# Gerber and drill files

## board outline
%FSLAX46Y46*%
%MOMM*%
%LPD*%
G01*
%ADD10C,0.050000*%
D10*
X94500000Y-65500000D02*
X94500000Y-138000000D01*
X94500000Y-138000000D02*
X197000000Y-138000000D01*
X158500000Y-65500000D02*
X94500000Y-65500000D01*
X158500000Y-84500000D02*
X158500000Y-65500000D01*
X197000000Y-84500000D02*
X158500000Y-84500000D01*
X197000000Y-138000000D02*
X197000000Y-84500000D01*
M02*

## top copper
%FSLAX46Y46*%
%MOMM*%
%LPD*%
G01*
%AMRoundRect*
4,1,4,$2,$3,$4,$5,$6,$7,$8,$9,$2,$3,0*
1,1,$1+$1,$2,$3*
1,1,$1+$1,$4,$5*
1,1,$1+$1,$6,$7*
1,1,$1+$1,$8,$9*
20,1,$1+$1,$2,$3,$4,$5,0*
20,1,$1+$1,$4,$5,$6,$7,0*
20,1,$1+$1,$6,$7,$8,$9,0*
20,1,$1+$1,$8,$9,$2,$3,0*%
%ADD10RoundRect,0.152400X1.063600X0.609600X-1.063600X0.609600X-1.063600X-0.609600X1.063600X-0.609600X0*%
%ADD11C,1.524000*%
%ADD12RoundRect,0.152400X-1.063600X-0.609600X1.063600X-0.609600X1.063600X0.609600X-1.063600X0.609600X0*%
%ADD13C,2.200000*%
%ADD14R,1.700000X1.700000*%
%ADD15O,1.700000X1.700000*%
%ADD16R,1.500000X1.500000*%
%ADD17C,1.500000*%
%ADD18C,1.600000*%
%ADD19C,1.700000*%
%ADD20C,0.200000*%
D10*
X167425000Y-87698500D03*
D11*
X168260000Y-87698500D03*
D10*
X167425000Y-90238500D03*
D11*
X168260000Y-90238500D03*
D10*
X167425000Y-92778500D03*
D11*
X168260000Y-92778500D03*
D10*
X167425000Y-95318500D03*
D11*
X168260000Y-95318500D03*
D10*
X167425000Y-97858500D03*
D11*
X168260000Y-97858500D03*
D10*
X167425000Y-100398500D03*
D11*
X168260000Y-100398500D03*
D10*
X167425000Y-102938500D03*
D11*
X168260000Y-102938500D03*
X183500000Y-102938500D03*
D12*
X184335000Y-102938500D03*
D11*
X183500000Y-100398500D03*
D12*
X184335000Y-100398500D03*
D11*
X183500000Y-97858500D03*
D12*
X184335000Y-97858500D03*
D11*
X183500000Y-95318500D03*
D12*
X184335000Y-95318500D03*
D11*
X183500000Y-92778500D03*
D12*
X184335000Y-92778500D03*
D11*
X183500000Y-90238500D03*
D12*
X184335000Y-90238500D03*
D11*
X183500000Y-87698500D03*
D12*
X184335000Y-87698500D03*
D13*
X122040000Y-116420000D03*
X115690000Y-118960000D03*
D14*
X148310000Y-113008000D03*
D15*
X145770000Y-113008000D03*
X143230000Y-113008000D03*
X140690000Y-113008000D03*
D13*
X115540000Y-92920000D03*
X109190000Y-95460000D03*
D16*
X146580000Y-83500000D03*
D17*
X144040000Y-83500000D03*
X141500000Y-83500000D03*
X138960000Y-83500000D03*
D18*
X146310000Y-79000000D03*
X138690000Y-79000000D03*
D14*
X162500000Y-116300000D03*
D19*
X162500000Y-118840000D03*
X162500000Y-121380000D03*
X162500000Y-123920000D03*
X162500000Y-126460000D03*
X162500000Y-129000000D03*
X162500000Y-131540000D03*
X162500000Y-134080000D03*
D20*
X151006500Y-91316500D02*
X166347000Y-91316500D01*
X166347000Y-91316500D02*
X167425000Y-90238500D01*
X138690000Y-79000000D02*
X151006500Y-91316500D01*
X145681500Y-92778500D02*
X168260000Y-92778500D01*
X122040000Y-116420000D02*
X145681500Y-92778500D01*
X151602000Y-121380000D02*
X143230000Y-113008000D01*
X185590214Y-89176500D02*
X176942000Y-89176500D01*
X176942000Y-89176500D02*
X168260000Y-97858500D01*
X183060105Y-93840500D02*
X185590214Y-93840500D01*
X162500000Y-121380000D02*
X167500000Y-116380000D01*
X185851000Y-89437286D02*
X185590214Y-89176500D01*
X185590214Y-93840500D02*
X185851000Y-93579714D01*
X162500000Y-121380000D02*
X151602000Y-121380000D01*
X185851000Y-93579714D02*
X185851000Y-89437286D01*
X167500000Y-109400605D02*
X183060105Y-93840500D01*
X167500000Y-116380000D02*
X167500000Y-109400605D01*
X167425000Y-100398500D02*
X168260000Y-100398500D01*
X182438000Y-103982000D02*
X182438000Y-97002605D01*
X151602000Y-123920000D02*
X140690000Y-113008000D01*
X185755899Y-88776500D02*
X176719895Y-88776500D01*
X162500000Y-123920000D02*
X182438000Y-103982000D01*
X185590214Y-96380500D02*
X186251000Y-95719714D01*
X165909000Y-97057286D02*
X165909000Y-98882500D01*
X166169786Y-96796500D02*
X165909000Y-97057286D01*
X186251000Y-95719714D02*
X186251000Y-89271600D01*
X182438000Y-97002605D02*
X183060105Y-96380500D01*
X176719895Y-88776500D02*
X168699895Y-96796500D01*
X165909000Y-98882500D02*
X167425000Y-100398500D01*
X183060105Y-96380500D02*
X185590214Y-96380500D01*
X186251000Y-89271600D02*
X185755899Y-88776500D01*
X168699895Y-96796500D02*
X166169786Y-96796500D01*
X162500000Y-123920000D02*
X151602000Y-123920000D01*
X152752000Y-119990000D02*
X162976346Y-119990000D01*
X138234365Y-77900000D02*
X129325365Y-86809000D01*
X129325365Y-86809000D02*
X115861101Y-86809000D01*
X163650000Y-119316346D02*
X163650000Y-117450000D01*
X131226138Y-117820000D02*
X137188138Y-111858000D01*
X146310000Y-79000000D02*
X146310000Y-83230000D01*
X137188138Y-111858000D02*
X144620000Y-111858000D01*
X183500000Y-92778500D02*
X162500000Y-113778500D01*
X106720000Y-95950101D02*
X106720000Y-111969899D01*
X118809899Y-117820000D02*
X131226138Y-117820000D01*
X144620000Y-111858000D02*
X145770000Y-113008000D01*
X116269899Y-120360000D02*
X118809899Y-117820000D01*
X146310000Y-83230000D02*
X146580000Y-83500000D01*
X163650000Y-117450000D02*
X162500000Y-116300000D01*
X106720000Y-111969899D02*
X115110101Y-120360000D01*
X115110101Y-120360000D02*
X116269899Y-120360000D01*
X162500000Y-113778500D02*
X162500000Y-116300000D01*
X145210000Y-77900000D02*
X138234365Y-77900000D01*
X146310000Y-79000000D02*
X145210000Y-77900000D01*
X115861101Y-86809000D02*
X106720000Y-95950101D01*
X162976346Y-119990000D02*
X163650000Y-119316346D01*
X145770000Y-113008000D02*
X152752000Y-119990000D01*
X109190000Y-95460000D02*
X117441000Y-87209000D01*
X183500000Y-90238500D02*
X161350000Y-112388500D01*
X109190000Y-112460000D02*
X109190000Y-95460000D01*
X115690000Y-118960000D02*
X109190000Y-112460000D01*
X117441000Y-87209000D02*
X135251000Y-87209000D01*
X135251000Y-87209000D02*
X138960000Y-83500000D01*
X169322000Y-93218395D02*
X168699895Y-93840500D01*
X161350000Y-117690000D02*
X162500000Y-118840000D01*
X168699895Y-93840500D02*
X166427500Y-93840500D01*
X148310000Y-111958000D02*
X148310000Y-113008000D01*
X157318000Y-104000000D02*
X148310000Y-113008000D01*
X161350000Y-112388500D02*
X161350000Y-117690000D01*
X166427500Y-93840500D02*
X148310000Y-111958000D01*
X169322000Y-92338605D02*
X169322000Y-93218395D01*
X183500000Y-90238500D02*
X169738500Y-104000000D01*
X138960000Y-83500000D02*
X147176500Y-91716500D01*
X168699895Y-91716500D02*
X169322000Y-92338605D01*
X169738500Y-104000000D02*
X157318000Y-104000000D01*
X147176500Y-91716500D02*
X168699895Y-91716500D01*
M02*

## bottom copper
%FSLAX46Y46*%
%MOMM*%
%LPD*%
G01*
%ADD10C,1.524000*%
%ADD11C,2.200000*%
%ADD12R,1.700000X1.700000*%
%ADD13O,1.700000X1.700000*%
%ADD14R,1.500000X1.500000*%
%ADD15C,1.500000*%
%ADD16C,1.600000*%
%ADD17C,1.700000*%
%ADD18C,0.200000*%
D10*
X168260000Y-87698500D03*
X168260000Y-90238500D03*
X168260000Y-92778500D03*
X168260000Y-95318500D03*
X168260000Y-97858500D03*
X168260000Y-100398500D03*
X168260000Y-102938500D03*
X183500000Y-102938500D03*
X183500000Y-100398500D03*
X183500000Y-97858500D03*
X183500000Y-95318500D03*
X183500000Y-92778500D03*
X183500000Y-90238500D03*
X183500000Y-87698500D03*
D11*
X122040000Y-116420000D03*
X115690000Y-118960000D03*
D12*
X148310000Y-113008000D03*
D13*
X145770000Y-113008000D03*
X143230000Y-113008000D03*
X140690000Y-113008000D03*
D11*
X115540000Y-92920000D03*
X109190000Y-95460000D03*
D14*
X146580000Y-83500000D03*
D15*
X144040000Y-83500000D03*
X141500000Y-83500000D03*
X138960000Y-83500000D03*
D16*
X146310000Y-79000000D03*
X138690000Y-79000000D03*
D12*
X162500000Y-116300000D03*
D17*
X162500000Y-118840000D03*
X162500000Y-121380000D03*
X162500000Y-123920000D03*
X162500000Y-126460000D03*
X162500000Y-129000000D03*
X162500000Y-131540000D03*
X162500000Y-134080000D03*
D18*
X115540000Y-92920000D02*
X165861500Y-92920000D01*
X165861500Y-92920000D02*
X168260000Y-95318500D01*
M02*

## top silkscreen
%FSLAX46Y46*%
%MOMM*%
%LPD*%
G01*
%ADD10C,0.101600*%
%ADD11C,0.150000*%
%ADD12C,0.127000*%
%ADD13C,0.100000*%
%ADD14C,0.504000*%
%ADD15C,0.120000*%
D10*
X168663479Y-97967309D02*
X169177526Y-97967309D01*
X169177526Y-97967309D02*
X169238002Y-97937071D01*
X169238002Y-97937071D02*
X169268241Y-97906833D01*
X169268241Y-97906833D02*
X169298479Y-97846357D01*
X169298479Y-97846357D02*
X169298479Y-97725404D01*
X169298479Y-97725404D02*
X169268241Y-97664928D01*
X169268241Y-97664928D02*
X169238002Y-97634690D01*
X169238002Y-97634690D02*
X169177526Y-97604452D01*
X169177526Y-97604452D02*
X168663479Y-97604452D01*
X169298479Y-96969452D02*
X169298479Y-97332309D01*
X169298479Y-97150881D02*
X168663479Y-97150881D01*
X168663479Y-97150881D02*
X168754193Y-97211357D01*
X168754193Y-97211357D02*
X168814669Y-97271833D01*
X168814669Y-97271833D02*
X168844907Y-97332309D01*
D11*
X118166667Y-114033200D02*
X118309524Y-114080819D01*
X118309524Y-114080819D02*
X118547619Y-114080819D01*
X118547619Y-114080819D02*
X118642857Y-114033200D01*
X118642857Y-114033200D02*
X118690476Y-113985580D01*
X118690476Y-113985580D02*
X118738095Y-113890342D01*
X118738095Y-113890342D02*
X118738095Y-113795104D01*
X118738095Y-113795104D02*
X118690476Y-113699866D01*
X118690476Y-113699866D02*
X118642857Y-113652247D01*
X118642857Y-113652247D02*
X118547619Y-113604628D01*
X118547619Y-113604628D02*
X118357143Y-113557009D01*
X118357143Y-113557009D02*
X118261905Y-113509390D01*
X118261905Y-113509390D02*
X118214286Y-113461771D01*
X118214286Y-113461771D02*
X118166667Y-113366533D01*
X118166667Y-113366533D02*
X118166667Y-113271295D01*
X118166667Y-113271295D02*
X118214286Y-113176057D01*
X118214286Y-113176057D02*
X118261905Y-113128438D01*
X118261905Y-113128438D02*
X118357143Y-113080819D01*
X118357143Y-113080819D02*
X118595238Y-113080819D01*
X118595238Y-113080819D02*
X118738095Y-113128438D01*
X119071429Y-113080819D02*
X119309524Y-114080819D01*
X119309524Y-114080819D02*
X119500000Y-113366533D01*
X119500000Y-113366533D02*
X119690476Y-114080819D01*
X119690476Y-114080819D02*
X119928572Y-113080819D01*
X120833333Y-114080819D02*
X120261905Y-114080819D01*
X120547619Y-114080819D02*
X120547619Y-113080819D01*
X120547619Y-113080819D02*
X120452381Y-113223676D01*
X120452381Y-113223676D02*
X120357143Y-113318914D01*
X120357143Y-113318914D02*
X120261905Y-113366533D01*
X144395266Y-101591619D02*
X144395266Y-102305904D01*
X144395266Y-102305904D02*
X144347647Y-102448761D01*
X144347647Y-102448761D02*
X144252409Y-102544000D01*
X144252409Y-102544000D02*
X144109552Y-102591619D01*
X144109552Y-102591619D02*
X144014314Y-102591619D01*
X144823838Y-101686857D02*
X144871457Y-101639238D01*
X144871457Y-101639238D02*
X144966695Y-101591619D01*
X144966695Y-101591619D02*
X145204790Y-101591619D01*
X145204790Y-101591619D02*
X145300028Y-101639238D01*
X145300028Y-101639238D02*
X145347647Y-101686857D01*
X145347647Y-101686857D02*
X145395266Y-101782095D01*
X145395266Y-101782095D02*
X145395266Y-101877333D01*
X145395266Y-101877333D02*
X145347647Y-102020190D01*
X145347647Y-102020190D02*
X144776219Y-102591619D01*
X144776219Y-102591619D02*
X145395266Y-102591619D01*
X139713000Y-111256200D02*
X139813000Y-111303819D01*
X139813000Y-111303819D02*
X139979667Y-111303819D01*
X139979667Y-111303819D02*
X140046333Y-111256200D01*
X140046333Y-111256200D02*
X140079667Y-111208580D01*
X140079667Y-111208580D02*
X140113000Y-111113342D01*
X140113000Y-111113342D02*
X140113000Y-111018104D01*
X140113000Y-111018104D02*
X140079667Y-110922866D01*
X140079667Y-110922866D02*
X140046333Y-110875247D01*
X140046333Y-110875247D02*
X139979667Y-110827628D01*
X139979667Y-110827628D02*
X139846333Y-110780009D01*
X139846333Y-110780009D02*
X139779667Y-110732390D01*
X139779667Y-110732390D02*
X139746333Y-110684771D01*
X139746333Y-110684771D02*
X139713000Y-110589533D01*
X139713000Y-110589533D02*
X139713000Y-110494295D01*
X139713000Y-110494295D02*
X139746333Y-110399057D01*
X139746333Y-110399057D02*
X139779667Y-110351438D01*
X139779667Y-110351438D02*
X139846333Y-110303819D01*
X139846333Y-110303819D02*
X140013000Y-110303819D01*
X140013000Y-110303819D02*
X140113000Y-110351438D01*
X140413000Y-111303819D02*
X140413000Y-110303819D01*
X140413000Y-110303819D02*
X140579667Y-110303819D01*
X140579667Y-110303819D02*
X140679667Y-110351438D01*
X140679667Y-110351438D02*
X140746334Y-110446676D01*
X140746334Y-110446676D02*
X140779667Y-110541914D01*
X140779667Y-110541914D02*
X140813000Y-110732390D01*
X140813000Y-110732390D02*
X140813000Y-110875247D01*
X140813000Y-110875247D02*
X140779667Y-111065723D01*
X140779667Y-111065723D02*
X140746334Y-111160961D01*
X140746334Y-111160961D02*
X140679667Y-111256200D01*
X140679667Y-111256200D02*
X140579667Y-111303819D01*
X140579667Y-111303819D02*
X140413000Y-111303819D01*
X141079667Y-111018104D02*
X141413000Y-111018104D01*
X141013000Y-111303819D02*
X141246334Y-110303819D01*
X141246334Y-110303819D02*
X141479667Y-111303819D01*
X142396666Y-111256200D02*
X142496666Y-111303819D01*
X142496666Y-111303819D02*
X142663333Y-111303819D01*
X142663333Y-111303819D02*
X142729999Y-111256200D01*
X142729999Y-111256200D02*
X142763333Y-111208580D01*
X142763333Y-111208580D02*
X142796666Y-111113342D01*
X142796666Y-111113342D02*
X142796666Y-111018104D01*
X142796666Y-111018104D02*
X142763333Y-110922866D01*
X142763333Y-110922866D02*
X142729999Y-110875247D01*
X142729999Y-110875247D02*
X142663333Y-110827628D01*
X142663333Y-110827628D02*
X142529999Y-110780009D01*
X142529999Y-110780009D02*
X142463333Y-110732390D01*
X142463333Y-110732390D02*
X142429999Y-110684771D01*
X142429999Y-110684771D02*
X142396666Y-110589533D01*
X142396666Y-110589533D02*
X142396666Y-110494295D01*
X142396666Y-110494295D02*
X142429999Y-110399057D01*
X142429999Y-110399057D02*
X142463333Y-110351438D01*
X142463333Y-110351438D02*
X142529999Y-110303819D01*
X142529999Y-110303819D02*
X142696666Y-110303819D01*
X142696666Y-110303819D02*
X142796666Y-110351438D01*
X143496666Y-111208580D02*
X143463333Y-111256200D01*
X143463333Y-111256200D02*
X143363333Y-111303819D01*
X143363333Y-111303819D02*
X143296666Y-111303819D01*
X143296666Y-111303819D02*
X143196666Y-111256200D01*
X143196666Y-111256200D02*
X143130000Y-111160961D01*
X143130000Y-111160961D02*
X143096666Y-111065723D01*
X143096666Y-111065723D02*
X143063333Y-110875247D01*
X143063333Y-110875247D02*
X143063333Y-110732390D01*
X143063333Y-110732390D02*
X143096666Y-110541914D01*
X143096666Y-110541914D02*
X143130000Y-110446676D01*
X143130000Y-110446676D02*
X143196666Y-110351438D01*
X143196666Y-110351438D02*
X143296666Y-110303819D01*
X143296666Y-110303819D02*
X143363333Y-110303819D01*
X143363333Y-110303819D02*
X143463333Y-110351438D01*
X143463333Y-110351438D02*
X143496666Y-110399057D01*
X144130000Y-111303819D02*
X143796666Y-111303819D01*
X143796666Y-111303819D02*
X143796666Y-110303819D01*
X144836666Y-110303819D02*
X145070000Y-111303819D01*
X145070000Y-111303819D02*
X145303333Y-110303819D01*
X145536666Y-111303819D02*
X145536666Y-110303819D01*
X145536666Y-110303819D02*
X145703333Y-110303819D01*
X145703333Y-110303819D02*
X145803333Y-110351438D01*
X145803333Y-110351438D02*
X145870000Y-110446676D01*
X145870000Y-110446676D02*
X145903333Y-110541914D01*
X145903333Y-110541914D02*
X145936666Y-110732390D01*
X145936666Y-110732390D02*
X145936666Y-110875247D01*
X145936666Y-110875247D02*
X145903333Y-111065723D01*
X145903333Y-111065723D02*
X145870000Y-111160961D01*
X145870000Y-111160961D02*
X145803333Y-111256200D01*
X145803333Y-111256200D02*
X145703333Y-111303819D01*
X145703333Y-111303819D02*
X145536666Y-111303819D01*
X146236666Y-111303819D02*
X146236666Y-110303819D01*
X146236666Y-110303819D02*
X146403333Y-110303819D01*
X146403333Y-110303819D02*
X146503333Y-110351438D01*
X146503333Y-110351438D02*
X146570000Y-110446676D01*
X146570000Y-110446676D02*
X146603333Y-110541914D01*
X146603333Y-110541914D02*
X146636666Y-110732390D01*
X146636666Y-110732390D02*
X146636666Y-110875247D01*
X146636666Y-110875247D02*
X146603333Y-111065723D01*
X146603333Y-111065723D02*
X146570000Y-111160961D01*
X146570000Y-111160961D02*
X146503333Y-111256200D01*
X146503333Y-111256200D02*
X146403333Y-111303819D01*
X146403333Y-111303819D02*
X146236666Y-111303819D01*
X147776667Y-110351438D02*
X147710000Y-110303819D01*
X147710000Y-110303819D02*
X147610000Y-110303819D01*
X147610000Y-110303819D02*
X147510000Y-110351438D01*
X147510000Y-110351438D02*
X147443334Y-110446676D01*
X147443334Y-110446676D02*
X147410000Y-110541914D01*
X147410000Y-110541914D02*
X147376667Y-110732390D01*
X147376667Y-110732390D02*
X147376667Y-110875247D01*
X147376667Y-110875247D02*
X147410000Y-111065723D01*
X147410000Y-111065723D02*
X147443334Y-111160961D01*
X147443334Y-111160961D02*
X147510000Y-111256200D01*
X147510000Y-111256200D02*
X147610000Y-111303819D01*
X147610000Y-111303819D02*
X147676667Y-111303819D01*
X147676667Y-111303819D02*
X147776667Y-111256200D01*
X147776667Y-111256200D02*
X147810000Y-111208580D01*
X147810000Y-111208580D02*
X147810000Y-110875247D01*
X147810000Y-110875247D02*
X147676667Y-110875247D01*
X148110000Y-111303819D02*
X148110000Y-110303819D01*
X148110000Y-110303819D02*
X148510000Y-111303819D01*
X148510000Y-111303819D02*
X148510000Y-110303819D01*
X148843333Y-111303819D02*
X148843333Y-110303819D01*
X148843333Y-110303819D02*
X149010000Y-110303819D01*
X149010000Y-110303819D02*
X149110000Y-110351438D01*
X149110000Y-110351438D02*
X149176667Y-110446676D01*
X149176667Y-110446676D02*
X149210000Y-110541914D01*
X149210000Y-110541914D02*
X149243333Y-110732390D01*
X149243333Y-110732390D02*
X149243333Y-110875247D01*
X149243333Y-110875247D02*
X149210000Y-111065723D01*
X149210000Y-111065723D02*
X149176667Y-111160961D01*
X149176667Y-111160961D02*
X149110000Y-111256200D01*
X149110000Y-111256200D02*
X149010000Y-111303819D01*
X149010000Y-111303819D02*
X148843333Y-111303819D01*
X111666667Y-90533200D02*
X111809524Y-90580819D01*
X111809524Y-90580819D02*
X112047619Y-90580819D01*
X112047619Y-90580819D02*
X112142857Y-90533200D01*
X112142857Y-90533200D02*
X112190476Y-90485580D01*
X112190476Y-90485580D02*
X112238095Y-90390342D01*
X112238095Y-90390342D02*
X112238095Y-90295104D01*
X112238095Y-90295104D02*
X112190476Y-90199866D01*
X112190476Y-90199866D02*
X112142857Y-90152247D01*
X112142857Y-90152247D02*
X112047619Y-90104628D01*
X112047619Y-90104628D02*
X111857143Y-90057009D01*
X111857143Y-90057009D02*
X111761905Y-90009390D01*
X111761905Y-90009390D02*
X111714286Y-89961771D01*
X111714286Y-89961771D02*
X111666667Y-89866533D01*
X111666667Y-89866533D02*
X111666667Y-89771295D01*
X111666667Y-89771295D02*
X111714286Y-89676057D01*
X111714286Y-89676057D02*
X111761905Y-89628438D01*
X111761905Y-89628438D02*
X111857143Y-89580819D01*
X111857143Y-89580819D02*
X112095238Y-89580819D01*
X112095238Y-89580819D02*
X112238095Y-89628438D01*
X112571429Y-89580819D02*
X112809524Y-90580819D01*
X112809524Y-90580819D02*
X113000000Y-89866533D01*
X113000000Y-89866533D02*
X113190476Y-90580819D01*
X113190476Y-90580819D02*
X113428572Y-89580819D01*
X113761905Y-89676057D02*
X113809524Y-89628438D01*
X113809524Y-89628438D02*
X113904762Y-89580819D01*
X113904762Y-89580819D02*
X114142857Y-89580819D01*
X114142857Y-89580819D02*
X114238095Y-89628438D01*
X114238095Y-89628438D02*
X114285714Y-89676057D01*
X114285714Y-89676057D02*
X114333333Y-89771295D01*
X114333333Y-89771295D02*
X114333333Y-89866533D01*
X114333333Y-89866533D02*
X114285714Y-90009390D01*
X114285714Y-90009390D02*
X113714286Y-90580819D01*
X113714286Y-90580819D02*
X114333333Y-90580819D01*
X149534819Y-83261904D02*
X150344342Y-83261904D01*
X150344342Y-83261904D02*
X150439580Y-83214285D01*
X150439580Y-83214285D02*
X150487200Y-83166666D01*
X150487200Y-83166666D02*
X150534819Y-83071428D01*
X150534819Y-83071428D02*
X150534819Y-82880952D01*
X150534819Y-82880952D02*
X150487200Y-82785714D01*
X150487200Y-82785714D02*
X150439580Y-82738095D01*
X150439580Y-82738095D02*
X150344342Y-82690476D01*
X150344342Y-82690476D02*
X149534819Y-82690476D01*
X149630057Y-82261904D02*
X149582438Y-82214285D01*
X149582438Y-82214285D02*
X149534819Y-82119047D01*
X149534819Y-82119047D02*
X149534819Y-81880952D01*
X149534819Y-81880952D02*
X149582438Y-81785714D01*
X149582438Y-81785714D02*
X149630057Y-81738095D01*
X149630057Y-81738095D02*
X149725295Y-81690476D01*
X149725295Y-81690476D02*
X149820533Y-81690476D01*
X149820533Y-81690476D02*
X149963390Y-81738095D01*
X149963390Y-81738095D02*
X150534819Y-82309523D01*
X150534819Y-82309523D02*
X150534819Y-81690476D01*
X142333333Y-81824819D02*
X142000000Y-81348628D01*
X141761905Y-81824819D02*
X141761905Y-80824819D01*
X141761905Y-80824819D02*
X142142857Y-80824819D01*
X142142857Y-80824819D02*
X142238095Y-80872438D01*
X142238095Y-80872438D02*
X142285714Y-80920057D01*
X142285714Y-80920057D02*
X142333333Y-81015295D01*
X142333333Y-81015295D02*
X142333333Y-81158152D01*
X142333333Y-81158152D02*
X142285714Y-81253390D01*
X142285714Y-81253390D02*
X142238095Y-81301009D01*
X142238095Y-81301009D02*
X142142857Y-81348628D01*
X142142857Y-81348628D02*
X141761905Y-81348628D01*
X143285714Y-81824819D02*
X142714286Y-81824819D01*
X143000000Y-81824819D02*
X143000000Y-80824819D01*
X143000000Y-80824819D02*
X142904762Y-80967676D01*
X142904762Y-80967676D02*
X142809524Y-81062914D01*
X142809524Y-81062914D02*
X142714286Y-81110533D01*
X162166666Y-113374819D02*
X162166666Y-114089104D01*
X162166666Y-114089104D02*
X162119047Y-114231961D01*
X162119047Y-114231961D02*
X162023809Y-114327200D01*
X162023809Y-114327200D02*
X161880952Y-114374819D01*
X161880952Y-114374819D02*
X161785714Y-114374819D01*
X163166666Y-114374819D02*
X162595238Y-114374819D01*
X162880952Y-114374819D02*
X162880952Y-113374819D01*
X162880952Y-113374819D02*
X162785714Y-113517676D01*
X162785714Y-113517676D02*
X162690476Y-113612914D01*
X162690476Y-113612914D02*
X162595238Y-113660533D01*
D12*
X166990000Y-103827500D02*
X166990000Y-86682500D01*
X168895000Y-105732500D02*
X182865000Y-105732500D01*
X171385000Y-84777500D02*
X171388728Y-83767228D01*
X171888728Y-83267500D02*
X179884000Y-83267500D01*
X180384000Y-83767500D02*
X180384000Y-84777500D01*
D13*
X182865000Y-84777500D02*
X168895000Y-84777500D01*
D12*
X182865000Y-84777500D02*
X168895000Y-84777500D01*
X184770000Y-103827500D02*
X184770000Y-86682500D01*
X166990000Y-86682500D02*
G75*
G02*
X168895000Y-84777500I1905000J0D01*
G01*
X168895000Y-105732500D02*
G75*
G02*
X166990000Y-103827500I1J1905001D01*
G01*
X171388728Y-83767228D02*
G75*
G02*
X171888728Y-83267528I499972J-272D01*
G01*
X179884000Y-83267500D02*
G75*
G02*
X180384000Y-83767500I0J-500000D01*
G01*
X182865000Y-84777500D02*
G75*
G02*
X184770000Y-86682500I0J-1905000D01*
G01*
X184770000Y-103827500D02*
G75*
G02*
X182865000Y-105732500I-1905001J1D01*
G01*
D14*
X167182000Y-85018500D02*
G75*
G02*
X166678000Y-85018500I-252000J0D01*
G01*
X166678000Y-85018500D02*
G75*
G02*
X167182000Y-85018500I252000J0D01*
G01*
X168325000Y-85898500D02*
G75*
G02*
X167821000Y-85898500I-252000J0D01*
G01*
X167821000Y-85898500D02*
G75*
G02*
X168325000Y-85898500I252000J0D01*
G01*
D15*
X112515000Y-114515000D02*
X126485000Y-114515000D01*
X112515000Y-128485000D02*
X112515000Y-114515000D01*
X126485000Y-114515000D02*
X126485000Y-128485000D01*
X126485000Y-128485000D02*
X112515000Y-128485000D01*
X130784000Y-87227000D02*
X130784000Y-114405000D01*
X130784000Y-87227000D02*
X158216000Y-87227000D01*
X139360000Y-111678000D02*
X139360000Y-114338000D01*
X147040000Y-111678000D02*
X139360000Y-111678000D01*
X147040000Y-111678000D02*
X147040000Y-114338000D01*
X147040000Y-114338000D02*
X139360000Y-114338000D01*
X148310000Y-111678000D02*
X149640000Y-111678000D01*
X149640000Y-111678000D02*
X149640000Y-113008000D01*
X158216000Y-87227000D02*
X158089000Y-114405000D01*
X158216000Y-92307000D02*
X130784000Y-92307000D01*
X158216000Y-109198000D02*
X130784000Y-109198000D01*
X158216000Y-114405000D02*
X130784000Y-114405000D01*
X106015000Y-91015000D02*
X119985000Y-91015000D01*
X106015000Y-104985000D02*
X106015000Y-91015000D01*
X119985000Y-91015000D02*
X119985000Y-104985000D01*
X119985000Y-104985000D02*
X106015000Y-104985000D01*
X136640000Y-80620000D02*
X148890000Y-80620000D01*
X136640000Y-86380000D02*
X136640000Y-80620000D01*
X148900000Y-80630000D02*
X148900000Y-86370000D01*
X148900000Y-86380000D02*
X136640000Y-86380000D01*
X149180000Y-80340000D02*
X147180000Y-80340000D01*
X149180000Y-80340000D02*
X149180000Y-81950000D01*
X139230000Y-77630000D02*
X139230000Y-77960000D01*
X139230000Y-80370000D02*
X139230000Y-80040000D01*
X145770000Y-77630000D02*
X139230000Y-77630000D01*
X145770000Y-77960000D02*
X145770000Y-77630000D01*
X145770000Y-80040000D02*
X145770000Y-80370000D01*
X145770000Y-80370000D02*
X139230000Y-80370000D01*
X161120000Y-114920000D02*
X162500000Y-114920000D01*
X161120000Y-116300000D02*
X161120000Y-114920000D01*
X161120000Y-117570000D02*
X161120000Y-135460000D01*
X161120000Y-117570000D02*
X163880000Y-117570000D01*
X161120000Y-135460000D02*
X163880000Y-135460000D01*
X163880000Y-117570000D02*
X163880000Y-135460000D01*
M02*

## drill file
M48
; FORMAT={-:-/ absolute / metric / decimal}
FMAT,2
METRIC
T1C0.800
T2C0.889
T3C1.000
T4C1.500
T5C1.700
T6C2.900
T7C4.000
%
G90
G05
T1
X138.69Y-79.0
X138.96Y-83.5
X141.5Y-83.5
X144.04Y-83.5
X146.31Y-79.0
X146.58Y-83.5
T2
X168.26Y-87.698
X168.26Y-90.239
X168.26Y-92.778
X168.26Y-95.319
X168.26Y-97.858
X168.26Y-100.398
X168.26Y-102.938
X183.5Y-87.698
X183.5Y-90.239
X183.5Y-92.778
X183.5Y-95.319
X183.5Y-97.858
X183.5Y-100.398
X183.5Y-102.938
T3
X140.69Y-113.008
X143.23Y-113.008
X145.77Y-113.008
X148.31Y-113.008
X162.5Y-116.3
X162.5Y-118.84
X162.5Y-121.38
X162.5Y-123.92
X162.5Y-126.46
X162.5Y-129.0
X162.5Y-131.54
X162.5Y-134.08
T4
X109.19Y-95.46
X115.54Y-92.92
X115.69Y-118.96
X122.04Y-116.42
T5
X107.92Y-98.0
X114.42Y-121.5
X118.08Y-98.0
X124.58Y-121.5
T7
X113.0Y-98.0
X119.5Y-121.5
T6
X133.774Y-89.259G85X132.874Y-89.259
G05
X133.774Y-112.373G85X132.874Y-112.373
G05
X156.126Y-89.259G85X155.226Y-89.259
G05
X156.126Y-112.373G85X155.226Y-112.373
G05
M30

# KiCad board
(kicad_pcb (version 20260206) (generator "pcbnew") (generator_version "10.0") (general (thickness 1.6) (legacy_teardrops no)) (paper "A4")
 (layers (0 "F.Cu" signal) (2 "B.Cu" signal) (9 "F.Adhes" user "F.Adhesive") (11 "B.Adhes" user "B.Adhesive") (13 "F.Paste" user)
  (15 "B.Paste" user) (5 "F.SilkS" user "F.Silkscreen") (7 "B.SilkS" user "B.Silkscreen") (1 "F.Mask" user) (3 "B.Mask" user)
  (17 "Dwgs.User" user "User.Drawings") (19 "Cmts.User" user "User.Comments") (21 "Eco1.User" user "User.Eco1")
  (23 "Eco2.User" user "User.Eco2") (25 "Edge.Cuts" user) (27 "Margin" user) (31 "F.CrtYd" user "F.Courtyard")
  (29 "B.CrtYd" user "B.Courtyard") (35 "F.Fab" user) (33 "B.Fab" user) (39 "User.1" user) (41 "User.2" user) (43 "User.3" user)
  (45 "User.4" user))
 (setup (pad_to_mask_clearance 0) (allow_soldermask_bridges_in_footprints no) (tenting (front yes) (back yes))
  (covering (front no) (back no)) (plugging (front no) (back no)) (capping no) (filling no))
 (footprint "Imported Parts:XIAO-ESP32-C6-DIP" (layer "F.Cu") (at 175.88 95.3185 90)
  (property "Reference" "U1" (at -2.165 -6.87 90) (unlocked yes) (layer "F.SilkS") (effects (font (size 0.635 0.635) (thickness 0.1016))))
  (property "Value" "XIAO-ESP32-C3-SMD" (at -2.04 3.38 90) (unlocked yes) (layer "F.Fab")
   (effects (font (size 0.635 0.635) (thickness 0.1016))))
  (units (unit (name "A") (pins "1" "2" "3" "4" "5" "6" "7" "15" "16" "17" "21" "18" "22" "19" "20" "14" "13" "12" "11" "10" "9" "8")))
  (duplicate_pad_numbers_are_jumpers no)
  (fp_line (start -8.509 -8.89) (end 8.636 -8.89) (stroke (width 0.127) (type solid)) (layer "F.SilkS"))
  (fp_line (start -10.414 -6.985) (end -10.414 6.985) (stroke (width 0.127) (type solid)) (layer "F.SilkS"))
  (fp_line (start 10.541 -4.495) (end 11.551272 -4.491272) (stroke (width 0.127) (type solid)) (layer "F.SilkS"))
  (fp_line (start 12.051 -3.991272) (end 12.051 4.004) (stroke (width 0.127) (type solid)) (layer "F.SilkS"))
  (fp_line (start 11.551 4.504) (end 10.541 4.504) (stroke (width 0.127) (type solid)) (layer "F.SilkS"))
  (fp_line (start 10.541 6.985) (end 10.541 -6.985) (stroke (width 0.1) (type solid)) (layer "F.SilkS"))
  (fp_line (start 10.541 6.985) (end 10.541 -6.985) (stroke (width 0.127) (type solid)) (layer "F.SilkS"))
  (fp_line (start -8.509 8.89) (end 8.636 8.89) (stroke (width 0.127) (type solid)) (layer "F.SilkS"))
  (fp_arc (start 8.636 -8.89) (mid 9.983038 -8.332038) (end 10.541 -6.985) (stroke (width 0.127) (type solid)) (layer "F.SilkS"))
  (fp_arc (start -10.414 -6.985) (mid -9.856038 -8.332038) (end -8.509 -8.89) (stroke (width 0.127) (type solid)) (layer "F.SilkS"))
  (fp_arc (start 11.551272 -4.491272) (mid 11.904644 -4.344724) (end 12.051 -3.991272) (stroke (width 0.127) (type default))
   (layer "F.SilkS"))
  (fp_arc (start 12.051 4.004) (mid 11.904553 4.357553) (end 11.551 4.504) (stroke (width 0.127) (type default)) (layer "F.SilkS"))
  (fp_arc (start 10.541 6.985) (mid 9.983038 8.332038) (end 8.636 8.89) (stroke (width 0.127) (type solid)) (layer "F.SilkS"))
  (fp_arc (start -8.509 8.89) (mid -9.856038 8.332038) (end -10.414 6.985) (stroke (width 0.127) (type solid)) (layer "F.SilkS"))
  (fp_circle (center 10.3 -8.95) (end 10.554 -8.95) (stroke (width 0.5) (type solid)) (fill yes) (layer "F.SilkS"))
  (fp_circle (center 9.42 -7.807) (end 9.674 -7.807) (stroke (width 0.5) (type solid)) (fill yes) (layer "F.SilkS"))
  (pad "1" smd roundrect (at 7.62 -8.455 180) (size 2.432 1.524) (layers "F.Cu" "F.Mask") (roundrect_rratio 0.1)
   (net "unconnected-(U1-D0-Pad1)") (thermal_bridge_angle 45))
  (pad "1" thru_hole circle (at 7.62 -7.62 180) (size 1.524 1.524) (drill 0.889) (layers "*.Cu" "*.Mask") (remove_unused_layers no)
   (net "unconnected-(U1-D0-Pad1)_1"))
  (pad "2" smd roundrect (at 5.08 -8.455 180) (size 2.432 1.524) (layers "F.Cu" "F.Mask") (roundrect_rratio 0.1) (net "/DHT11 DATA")
   (thermal_bridge_angle 45))
  (pad "2" thru_hole circle (at 5.08 -7.62 180) (size 1.524 1.524) (drill 0.889) (layers "*.Cu" "*.Mask") (remove_unused_layers no)
   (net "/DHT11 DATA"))
  (pad "3" smd roundrect (at 2.54 -8.455 180) (size 2.432 1.524) (layers "F.Cu" "F.Mask") (roundrect_rratio 0.1) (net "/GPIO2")
   (thermal_bridge_angle 45))
  (pad "3" thru_hole circle (at 2.54 -7.62 180) (size 1.524 1.524) (drill 0.889) (layers "*.Cu" "*.Mask") (remove_unused_layers no)
   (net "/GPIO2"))
  (pad "4" smd roundrect (at 0 -8.455 180) (size 2.432 1.524) (layers "F.Cu" "F.Mask") (roundrect_rratio 0.1) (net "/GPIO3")
   (thermal_bridge_angle 45))
  (pad "4" thru_hole circle (at 0 -7.62 180) (size 1.524 1.524) (drill 0.889) (layers "*.Cu" "*.Mask") (remove_unused_layers no)
   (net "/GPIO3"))
  (pad "5" smd roundrect (at -2.54 -8.455 180) (size 2.432 1.524) (layers "F.Cu" "F.Mask") (roundrect_rratio 0.1) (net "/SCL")
   (thermal_bridge_angle 45))
  (pad "5" thru_hole circle (at -2.54 -7.62 180) (size 1.524 1.524) (drill 0.889) (layers "*.Cu" "*.Mask") (remove_unused_layers no)
   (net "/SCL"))
  (pad "6" smd roundrect (at -5.08 -8.455 180) (size 2.432 1.524) (layers "F.Cu" "F.Mask") (roundrect_rratio 0.1) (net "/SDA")
   (thermal_bridge_angle 45))
  (pad "6" thru_hole circle (at -5.08 -7.62 180) (size 1.524 1.524) (drill 0.889) (layers "*.Cu" "*.Mask") (remove_unused_layers no)
   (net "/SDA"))
  (pad "7" smd roundrect (at -7.62 -8.455 180) (size 2.432 1.524) (layers "F.Cu" "F.Mask") (roundrect_rratio 0.1)
   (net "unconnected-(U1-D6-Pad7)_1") (thermal_bridge_angle 45))
  (pad "7" thru_hole circle (at -7.62 -7.62 180) (size 1.524 1.524) (drill 0.889) (layers "*.Cu" "*.Mask") (remove_unused_layers no)
   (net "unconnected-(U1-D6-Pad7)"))
  (pad "8" thru_hole circle (at -7.62 7.62) (size 1.524 1.524) (drill 0.889) (layers "*.Cu" "*.Mask") (remove_unused_layers no)
   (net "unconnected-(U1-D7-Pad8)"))
  (pad "8" smd roundrect (at -7.62 8.455) (size 2.432 1.524) (layers "F.Cu" "F.Mask") (roundrect_rratio 0.1)
   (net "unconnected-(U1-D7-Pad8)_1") (thermal_bridge_angle 45))
  (pad "9" thru_hole circle (at -5.08 7.62) (size 1.524 1.524) (drill 0.889) (layers "*.Cu" "*.Mask") (remove_unused_layers no)
   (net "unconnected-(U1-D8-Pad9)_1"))
  (pad "9" smd roundrect (at -5.08 8.455) (size 2.432 1.524) (layers "F.Cu" "F.Mask") (roundrect_rratio 0.1)
   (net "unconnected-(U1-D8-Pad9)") (thermal_bridge_angle 45))
  (pad "10" thru_hole circle (at -2.54 7.62) (size 1.524 1.524) (drill 0.889) (layers "*.Cu" "*.Mask") (remove_unused_layers no)
   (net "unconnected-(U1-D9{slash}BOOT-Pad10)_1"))
  (pad "10" smd roundrect (at -2.54 8.455) (size 2.432 1.524) (layers "F.Cu" "F.Mask") (roundrect_rratio 0.1)
   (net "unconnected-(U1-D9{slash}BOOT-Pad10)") (thermal_bridge_angle 45))
  (pad "11" thru_hole circle (at 0 7.62) (size 1.524 1.524) (drill 0.889) (layers "*.Cu" "*.Mask") (remove_unused_layers no)
   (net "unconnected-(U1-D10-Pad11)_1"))
  (pad "11" smd roundrect (at 0 8.455) (size 2.432 1.524) (layers "F.Cu" "F.Mask") (roundrect_rratio 0.1) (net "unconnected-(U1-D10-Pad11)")
   (thermal_bridge_angle 45))
  (pad "12" thru_hole circle (at 2.54 7.62) (size 1.524 1.524) (drill 0.889) (layers "*.Cu" "*.Mask") (remove_unused_layers no)
   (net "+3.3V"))
  (pad "12" smd roundrect (at 2.54 8.455) (size 2.432 1.524) (layers "F.Cu" "F.Mask") (roundrect_rratio 0.1) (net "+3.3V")
   (thermal_bridge_angle 45))
  (pad "13" thru_hole circle (at 5.08 7.62) (size 1.524 1.524) (drill 0.889) (layers "*.Cu" "*.Mask") (remove_unused_layers no) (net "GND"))
  (pad "13" smd roundrect (at 5.08 8.455) (size 2.432 1.524) (layers "F.Cu" "F.Mask") (roundrect_rratio 0.1) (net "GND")
   (thermal_bridge_angle 45))
  (pad "14" thru_hole circle (at 7.62 7.62) (size 1.524 1.524) (drill 0.889) (layers "*.Cu" "*.Mask") (remove_unused_layers no) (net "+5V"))
  (pad "14" smd roundrect (at 7.62 8.455) (size 2.432 1.524) (layers "F.Cu" "F.Mask") (roundrect_rratio 0.1) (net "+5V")
   (thermal_bridge_angle 45)))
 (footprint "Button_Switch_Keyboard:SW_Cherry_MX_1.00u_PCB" (layer "F.Cu") (at 122.04 116.42)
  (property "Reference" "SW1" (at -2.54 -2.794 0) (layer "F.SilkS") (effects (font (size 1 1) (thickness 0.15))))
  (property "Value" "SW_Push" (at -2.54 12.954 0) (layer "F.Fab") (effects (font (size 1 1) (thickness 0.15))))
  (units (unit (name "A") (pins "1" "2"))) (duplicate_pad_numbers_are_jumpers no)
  (fp_line (start -9.525 -1.905) (end 4.445 -1.905) (stroke (width 0.12) (type solid)) (layer "F.SilkS"))
  (fp_line (start -9.525 12.065) (end -9.525 -1.905) (stroke (width 0.12) (type solid)) (layer "F.SilkS"))
  (fp_line (start 4.445 -1.905) (end 4.445 12.065) (stroke (width 0.12) (type solid)) (layer "F.SilkS"))
  (fp_line (start 4.445 12.065) (end -9.525 12.065) (stroke (width 0.12) (type solid)) (layer "F.SilkS"))
  (pad "" np_thru_hole circle (at -7.62 5.08) (size 1.7 1.7) (drill 1.7) (layers "*.Cu" "*.Mask"))
  (pad "" np_thru_hole circle (at -2.54 5.08) (size 4 4) (drill 4) (layers "*.Cu" "*.Mask"))
  (pad "" np_thru_hole circle (at 2.54 5.08) (size 1.7 1.7) (drill 1.7) (layers "*.Cu" "*.Mask"))
  (pad "1" thru_hole circle (at 0 0) (size 2.2 2.2) (drill 1.5) (layers "*.Cu" "*.Mask") (remove_unused_layers no) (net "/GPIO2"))
  (pad "2" thru_hole circle (at -6.35 2.54) (size 2.2 2.2) (drill 1.5) (layers "*.Cu" "*.Mask") (remove_unused_layers no) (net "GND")))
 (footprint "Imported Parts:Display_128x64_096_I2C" (layer "F.Cu") (at 144.5 113.008 180)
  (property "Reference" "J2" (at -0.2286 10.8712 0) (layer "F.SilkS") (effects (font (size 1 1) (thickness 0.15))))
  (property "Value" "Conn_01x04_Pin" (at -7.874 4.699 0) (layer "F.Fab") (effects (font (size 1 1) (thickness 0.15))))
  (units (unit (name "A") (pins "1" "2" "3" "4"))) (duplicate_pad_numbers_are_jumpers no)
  (fp_line (start 13.716 25.781) (end 13.716 -1.397) (stroke (width 0.12) (type solid)) (layer "F.SilkS"))
  (fp_line (start 13.716 25.781) (end -13.716 25.781) (stroke (width 0.12) (type solid)) (layer "F.SilkS"))
  (fp_line (start 5.14 1.33) (end 5.14 -1.33) (stroke (width 0.12) (type solid)) (layer "F.SilkS"))
  (fp_line (start -2.54 1.33) (end 5.14 1.33) (stroke (width 0.12) (type solid)) (layer "F.SilkS"))
  (fp_line (start -2.54 1.33) (end -2.54 -1.33) (stroke (width 0.12) (type solid)) (layer "F.SilkS"))
  (fp_line (start -2.54 -1.33) (end 5.14 -1.33) (stroke (width 0.12) (type solid)) (layer "F.SilkS"))
  (fp_line (start -3.81 1.33) (end -5.14 1.33) (stroke (width 0.12) (type solid)) (layer "F.SilkS"))
  (fp_line (start -5.14 1.33) (end -5.14 0) (stroke (width 0.12) (type solid)) (layer "F.SilkS"))
  (fp_line (start -13.716 25.781) (end -13.589 -1.397) (stroke (width 0.12) (type solid)) (layer "F.SilkS"))
  (fp_line (start -13.716 20.701) (end 13.716 20.701) (stroke (width 0.12) (type solid)) (layer "F.SilkS"))
  (fp_line (start -13.716 3.81) (end 13.716 3.81) (stroke (width 0.12) (type solid)) (layer "F.SilkS"))
  (fp_line (start -13.716 -1.397) (end 13.716 -1.397) (stroke (width 0.12) (type solid)) (layer "F.SilkS"))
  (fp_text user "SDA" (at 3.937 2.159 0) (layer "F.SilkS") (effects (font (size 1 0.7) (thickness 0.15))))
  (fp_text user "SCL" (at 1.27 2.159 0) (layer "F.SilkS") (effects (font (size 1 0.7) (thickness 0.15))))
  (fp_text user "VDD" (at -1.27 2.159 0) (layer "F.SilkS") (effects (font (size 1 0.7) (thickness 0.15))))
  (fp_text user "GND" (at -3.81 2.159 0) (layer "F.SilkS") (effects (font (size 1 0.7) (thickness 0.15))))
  (pad "" np_thru_hole oval (at -11.176 0.635 180) (size 3.8 2.9) (drill oval 3.8 2.9) (layers "*.Cu" "*.Mask"))
  (pad "" np_thru_hole oval (at -11.176 23.749 180) (size 3.8 2.9) (drill oval 3.8 2.9) (layers "*.Cu" "*.Mask"))
  (pad "" np_thru_hole oval (at 11.176 0.635 180) (size 3.8 2.9) (drill oval 3.8 2.9) (layers "*.Cu" "*.Mask"))
  (pad "" np_thru_hole oval (at 11.176 23.749 180) (size 3.8 2.9) (drill oval 3.8 2.9) (layers "*.Cu" "*.Mask"))
  (pad "1" thru_hole rect (at -3.81 0 270) (size 1.7 1.7) (drill 1) (layers "*.Cu" "*.Mask") (remove_unused_layers no) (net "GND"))
  (pad "2" thru_hole oval (at -1.27 0 270) (size 1.7 1.7) (drill 1) (layers "*.Cu" "*.Mask") (remove_unused_layers no) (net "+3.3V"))
  (pad "3" thru_hole oval (at 1.27 0 270) (size 1.7 1.7) (drill 1) (layers "*.Cu" "*.Mask") (remove_unused_layers no) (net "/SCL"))
  (pad "4" thru_hole oval (at 3.81 0 270) (size 1.7 1.7) (drill 1) (layers "*.Cu" "*.Mask") (remove_unused_layers no) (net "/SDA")))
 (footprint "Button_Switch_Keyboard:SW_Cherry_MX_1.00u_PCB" (layer "F.Cu") (at 115.54 92.92)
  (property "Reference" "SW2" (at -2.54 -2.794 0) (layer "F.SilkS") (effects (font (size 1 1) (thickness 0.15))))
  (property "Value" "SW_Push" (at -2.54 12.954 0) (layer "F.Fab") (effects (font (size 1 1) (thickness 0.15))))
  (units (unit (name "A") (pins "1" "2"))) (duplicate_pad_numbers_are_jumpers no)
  (fp_line (start -9.525 -1.905) (end 4.445 -1.905) (stroke (width 0.12) (type solid)) (layer "F.SilkS"))
  (fp_line (start -9.525 12.065) (end -9.525 -1.905) (stroke (width 0.12) (type solid)) (layer "F.SilkS"))
  (fp_line (start 4.445 -1.905) (end 4.445 12.065) (stroke (width 0.12) (type solid)) (layer "F.SilkS"))
  (fp_line (start 4.445 12.065) (end -9.525 12.065) (stroke (width 0.12) (type solid)) (layer "F.SilkS"))
  (pad "" np_thru_hole circle (at -7.62 5.08) (size 1.7 1.7) (drill 1.7) (layers "*.Cu" "*.Mask"))
  (pad "" np_thru_hole circle (at -2.54 5.08) (size 4 4) (drill 4) (layers "*.Cu" "*.Mask"))
  (pad "" np_thru_hole circle (at 2.54 5.08) (size 1.7 1.7) (drill 1.7) (layers "*.Cu" "*.Mask"))
  (pad "1" thru_hole circle (at 0 0) (size 2.2 2.2) (drill 1.5) (layers "*.Cu" "*.Mask") (remove_unused_layers no) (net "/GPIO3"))
  (pad "2" thru_hole circle (at -6.35 2.54) (size 2.2 2.2) (drill 1.5) (layers "*.Cu" "*.Mask") (remove_unused_layers no) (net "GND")))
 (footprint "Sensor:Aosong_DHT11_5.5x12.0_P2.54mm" (layer "F.Cu") (at 146.58 83.5 -90)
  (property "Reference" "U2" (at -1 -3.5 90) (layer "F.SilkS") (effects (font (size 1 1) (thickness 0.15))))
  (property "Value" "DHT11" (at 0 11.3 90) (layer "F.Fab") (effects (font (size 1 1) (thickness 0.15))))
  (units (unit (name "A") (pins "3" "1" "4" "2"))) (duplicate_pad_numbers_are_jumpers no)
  (fp_line (start -2.88 9.94) (end -2.88 -2.31) (stroke (width 0.12) (type solid)) (layer "F.SilkS"))
  (fp_line (start 2.88 9.94) (end -2.88 9.94) (stroke (width 0.12) (type solid)) (layer "F.SilkS"))
  (fp_line (start -2.87 -2.32) (end 2.87 -2.32) (stroke (width 0.12) (type solid)) (layer "F.SilkS"))
  (fp_line (start 2.88 -2.32) (end 2.88 9.94) (stroke (width 0.12) (type solid)) (layer "F.SilkS"))
  (fp_line (start -3.16 -2.6) (end -3.16 -0.6) (stroke (width 0.12) (type solid)) (layer "F.SilkS"))
  (fp_line (start -3.16 -2.6) (end -1.55 -2.6) (stroke (width 0.12) (type solid)) (layer "F.SilkS"))
  (pad "1" thru_hole rect (at 0 0 270) (size 1.5 1.5) (drill 0.8) (layers "*.Cu" "*.Mask") (remove_unused_layers no) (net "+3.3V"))
  (pad "2" thru_hole circle (at 0 2.54 270) (size 1.5 1.5) (drill 0.8) (layers "*.Cu" "*.Mask") (remove_unused_layers no)
   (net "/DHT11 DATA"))
  (pad "3" thru_hole circle (at 0 5.08 270) (size 1.5 1.5) (drill 0.8) (layers "*.Cu" "*.Mask") (remove_unused_layers no)
   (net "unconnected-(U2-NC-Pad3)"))
  (pad "4" thru_hole circle (at 0 7.62 270) (size 1.5 1.5) (drill 0.8) (layers "*.Cu" "*.Mask") (remove_unused_layers no) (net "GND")))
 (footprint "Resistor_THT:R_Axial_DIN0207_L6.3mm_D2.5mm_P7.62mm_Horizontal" (layer "F.Cu") (at 146.31 79 180)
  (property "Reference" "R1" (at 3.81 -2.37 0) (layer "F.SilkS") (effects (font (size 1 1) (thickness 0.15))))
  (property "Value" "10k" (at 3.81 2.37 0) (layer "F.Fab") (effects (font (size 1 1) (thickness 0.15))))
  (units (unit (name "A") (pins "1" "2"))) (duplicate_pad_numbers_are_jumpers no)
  (fp_line (start 7.08 1.37) (end 7.08 1.04) (stroke (width 0.12) (type solid)) (layer "F.SilkS"))
  (fp_line (start 7.08 -1.37) (end 7.08 -1.04) (stroke (width 0.12) (type solid)) (layer "F.SilkS"))
  (fp_line (start 0.54 1.37) (end 7.08 1.37) (stroke (width 0.12) (type solid)) (layer "F.SilkS"))
  (fp_line (start 0.54 1.04) (end 0.54 1.37) (stroke (width 0.12) (type solid)) (layer "F.SilkS"))
  (fp_line (start 0.54 -1.04) (end 0.54 -1.37) (stroke (width 0.12) (type solid)) (layer "F.SilkS"))
  (fp_line (start 0.54 -1.37) (end 7.08 -1.37) (stroke (width 0.12) (type solid)) (layer "F.SilkS"))
  (pad "1" thru_hole circle (at 0 0 180) (size 1.6 1.6) (drill 0.8) (layers "*.Cu" "*.Mask") (remove_unused_layers no) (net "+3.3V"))
  (pad "2" thru_hole circle (at 7.62 0 180) (size 1.6 1.6) (drill 0.8) (layers "*.Cu" "*.Mask") (remove_unused_layers no)
   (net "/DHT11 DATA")))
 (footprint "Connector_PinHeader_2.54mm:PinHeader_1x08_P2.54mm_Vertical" (layer "F.Cu") (at 162.5 116.3)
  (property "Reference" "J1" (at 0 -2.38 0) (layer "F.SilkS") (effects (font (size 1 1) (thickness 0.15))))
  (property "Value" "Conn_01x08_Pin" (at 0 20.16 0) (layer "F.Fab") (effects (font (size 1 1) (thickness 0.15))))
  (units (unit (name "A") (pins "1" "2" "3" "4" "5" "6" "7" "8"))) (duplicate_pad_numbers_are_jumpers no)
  (fp_line (start -1.38 -1.38) (end 0 -1.38) (stroke (width 0.12) (type solid)) (layer "F.SilkS"))
  (fp_line (start -1.38 0) (end -1.38 -1.38) (stroke (width 0.12) (type solid)) (layer "F.SilkS"))
  (fp_line (start -1.38 1.27) (end -1.38 19.16) (stroke (width 0.12) (type solid)) (layer "F.SilkS"))
  (fp_line (start -1.38 1.27) (end 1.38 1.27) (stroke (width 0.12) (type solid)) (layer "F.SilkS"))
  (fp_line (start -1.38 19.16) (end 1.38 19.16) (stroke (width 0.12) (type solid)) (layer "F.SilkS"))
  (fp_line (start 1.38 1.27) (end 1.38 19.16) (stroke (width 0.12) (type solid)) (layer "F.SilkS"))
  (pad "1" thru_hole rect (at 0 0) (size 1.7 1.7) (drill 1) (layers "*.Cu" "*.Mask") (remove_unused_layers no) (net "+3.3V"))
  (pad "2" thru_hole circle (at 0 2.54) (size 1.7 1.7) (drill 1) (layers "*.Cu" "*.Mask") (remove_unused_layers no) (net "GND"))
  (pad "3" thru_hole circle (at 0 5.08) (size 1.7 1.7) (drill 1) (layers "*.Cu" "*.Mask") (remove_unused_layers no) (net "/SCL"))
  (pad "4" thru_hole circle (at 0 7.62) (size 1.7 1.7) (drill 1) (layers "*.Cu" "*.Mask") (remove_unused_layers no) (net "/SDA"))
  (pad "5" thru_hole circle (at 0 10.16) (size 1.7 1.7) (drill 1) (layers "*.Cu" "*.Mask") (remove_unused_layers no)
   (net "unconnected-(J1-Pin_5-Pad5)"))
  (pad "6" thru_hole circle (at 0 12.7) (size 1.7 1.7) (drill 1) (layers "*.Cu" "*.Mask") (remove_unused_layers no)
   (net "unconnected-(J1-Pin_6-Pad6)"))
  (pad "7" thru_hole circle (at 0 15.24) (size 1.7 1.7) (drill 1) (layers "*.Cu" "*.Mask") (remove_unused_layers no)
   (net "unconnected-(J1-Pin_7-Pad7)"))
  (pad "8" thru_hole circle (at 0 17.78) (size 1.7 1.7) (drill 1) (layers "*.Cu" "*.Mask") (remove_unused_layers no)
   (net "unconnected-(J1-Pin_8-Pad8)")))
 (gr_line (start 94.5 65.5) (end 94.5 138) (stroke (width 0.05) (type default)) (layer "Edge.Cuts"))
 (gr_line (start 94.5 138) (end 197 138) (stroke (width 0.05) (type default)) (layer "Edge.Cuts"))
 (gr_line (start 158.5 65.5) (end 94.5 65.5) (stroke (width 0.05) (type default)) (layer "Edge.Cuts"))
 (gr_line (start 158.5 84.5) (end 158.5 65.5) (stroke (width 0.05) (type default)) (layer "Edge.Cuts"))
 (gr_line (start 197 84.5) (end 158.5 84.5) (stroke (width 0.05) (type default)) (layer "Edge.Cuts"))
 (gr_line (start 197 138) (end 197 84.5) (stroke (width 0.05) (type default)) (layer "Edge.Cuts"))
 (segment (start 151.0065 91.3165) (end 166.347 91.3165) (width 0.2) (layer "F.Cu") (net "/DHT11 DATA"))
 (segment (start 166.347 91.3165) (end 167.425 90.2385) (width 0.2) (layer "F.Cu") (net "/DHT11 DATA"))
 (segment (start 138.69 79) (end 151.0065 91.3165) (width 0.2) (layer "F.Cu") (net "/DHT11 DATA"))
 (segment (start 145.6815 92.7785) (end 168.26 92.7785) (width 0.2) (layer "F.Cu") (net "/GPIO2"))
 (segment (start 122.04 116.42) (end 145.6815 92.7785) (width 0.2) (layer "F.Cu") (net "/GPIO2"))
 (segment (start 115.54 92.92) (end 165.8615 92.92) (width 0.2) (layer "B.Cu") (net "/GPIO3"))
 (segment (start 165.8615 92.92) (end 168.26 95.3185) (width 0.2) (layer "B.Cu") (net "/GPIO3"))
 (segment (start 151.602 121.38) (end 143.23 113.008) (width 0.2) (layer "F.Cu") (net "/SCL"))
 (segment (start 185.590214 89.1765) (end 176.942 89.1765) (width 0.2) (layer "F.Cu") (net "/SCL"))
 (segment (start 176.942 89.1765) (end 168.26 97.8585) (width 0.2) (layer "F.Cu") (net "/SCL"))
 (segment (start 183.060105 93.8405) (end 185.590214 93.8405) (width 0.2) (layer "F.Cu") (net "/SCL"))
 (segment (start 162.5 121.38) (end 167.5 116.38) (width 0.2) (layer "F.Cu") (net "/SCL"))
 (segment (start 185.851 89.437286) (end 185.590214 89.1765) (width 0.2) (layer "F.Cu") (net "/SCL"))
 (segment (start 185.590214 93.8405) (end 185.851 93.579714) (width 0.2) (layer "F.Cu") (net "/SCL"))
 (segment (start 162.5 121.38) (end 151.602 121.38) (width 0.2) (layer "F.Cu") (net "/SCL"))
 (segment (start 185.851 93.579714) (end 185.851 89.437286) (width 0.2) (layer "F.Cu") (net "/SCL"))
 (segment (start 167.5 109.400605) (end 183.060105 93.8405) (width 0.2) (layer "F.Cu") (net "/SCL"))
 (segment (start 167.5 116.38) (end 167.5 109.400605) (width 0.2) (layer "F.Cu") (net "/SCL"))
 (segment (start 167.425 100.3985) (end 168.26 100.3985) (width 0.2) (layer "F.Cu") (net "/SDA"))
 (segment (start 182.438 103.982) (end 182.438 97.002605) (width 0.2) (layer "F.Cu") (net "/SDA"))
 (segment (start 151.602 123.92) (end 140.69 113.008) (width 0.2) (layer "F.Cu") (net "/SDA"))
 (segment (start 185.755899 88.7765) (end 176.719895 88.7765) (width 0.2) (layer "F.Cu") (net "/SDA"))
 (segment (start 162.5 123.92) (end 182.438 103.982) (width 0.2) (layer "F.Cu") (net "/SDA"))
 (segment (start 185.590214 96.3805) (end 186.251 95.719714) (width 0.2) (layer "F.Cu") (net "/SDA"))
 (segment (start 165.909 97.057286) (end 165.909 98.8825) (width 0.2) (layer "F.Cu") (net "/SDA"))
 (segment (start 166.169786 96.7965) (end 165.909 97.057286) (width 0.2) (layer "F.Cu") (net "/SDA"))
 (segment (start 186.251 95.719714) (end 186.251 89.2716) (width 0.2) (layer "F.Cu") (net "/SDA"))
 (segment (start 182.438 97.002605) (end 183.060105 96.3805) (width 0.2) (layer "F.Cu") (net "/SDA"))
 (segment (start 176.719895 88.7765) (end 168.699895 96.7965) (width 0.2) (layer "F.Cu") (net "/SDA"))
 (segment (start 165.909 98.8825) (end 167.425 100.3985) (width 0.2) (layer "F.Cu") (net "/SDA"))
 (segment (start 183.060105 96.3805) (end 185.590214 96.3805) (width 0.2) (layer "F.Cu") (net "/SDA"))
 (segment (start 186.251 89.2716) (end 185.755899 88.7765) (width 0.2) (layer "F.Cu") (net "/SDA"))
 (segment (start 168.699895 96.7965) (end 166.169786 96.7965) (width 0.2) (layer "F.Cu") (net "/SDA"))
 (segment (start 162.5 123.92) (end 151.602 123.92) (width 0.2) (layer "F.Cu") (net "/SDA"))
 (segment (start 152.752 119.99) (end 162.976346 119.99) (width 0.2) (layer "F.Cu") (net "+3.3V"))
 (segment (start 138.234365 77.9) (end 129.325365 86.809) (width 0.2) (layer "F.Cu") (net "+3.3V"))
 (segment (start 129.325365 86.809) (end 115.861101 86.809) (width 0.2) (layer "F.Cu") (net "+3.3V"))
 (segment (start 163.65 119.316346) (end 163.65 117.45) (width 0.2) (layer "F.Cu") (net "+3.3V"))
 (segment (start 131.226138 117.82) (end 137.188138 111.858) (width 0.2) (layer "F.Cu") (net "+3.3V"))
 (segment (start 146.31 79) (end 146.31 83.23) (width 0.2) (layer "F.Cu") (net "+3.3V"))
 (segment (start 137.188138 111.858) (end 144.62 111.858) (width 0.2) (layer "F.Cu") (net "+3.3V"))
 (segment (start 183.5 92.7785) (end 162.5 113.7785) (width 0.2) (layer "F.Cu") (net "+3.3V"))
 (segment (start 106.72 95.950101) (end 106.72 111.969899) (width 0.2) (layer "F.Cu") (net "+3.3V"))
 (segment (start 118.809899 117.82) (end 131.226138 117.82) (width 0.2) (layer "F.Cu") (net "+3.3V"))
 (segment (start 144.62 111.858) (end 145.77 113.008) (width 0.2) (layer "F.Cu") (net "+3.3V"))
 (segment (start 116.269899 120.36) (end 118.809899 117.82) (width 0.2) (layer "F.Cu") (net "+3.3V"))
 (segment (start 146.31 83.23) (end 146.58 83.5) (width 0.2) (layer "F.Cu") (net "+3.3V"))
 (segment (start 163.65 117.45) (end 162.5 116.3) (width 0.2) (layer "F.Cu") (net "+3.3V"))
 (segment (start 106.72 111.969899) (end 115.110101 120.36) (width 0.2) (layer "F.Cu") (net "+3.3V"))
 (segment (start 115.110101 120.36) (end 116.269899 120.36) (width 0.2) (layer "F.Cu") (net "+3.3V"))
 (segment (start 162.5 113.7785) (end 162.5 116.3) (width 0.2) (layer "F.Cu") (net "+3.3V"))
 (segment (start 145.21 77.9) (end 138.234365 77.9) (width 0.2) (layer "F.Cu") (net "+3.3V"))
 (segment (start 146.31 79) (end 145.21 77.9) (width 0.2) (layer "F.Cu") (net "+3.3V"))
 (segment (start 115.861101 86.809) (end 106.72 95.950101) (width 0.2) (layer "F.Cu") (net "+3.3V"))
 (segment (start 162.976346 119.99) (end 163.65 119.316346) (width 0.2) (layer "F.Cu") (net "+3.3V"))
 (segment (start 145.77 113.008) (end 152.752 119.99) (width 0.2) (layer "F.Cu") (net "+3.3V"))
 (segment (start 109.19 95.46) (end 117.441 87.209) (width 0.2) (layer "F.Cu") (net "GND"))
 (segment (start 183.5 90.2385) (end 161.35 112.3885) (width 0.2) (layer "F.Cu") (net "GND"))
 (segment (start 109.19 112.46) (end 109.19 95.46) (width 0.2) (layer "F.Cu") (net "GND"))
 (segment (start 115.69 118.96) (end 109.19 112.46) (width 0.2) (layer "F.Cu") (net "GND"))
 (segment (start 117.441 87.209) (end 135.251 87.209) (width 0.2) (layer "F.Cu") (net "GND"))
 (segment (start 135.251 87.209) (end 138.96 83.5) (width 0.2) (layer "F.Cu") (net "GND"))
 (segment (start 169.322 93.218395) (end 168.699895 93.8405) (width 0.2) (layer "F.Cu") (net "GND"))
 (segment (start 161.35 117.69) (end 162.5 118.84) (width 0.2) (layer "F.Cu") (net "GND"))
 (segment (start 168.699895 93.8405) (end 166.4275 93.8405) (width 0.2) (layer "F.Cu") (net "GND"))
 (segment (start 148.31 111.958) (end 148.31 113.008) (width 0.2) (layer "F.Cu") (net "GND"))
 (segment (start 157.318 104) (end 148.31 113.008) (width 0.2) (layer "F.Cu") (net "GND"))
 (segment (start 161.35 112.3885) (end 161.35 117.69) (width 0.2) (layer "F.Cu") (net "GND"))
 (segment (start 166.4275 93.8405) (end 148.31 111.958) (width 0.2) (layer "F.Cu") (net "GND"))
 (segment (start 169.322 92.338605) (end 169.322 93.218395) (width 0.2) (layer "F.Cu") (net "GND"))
 (segment (start 183.5 90.2385) (end 169.7385 104) (width 0.2) (layer "F.Cu") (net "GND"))
 (segment (start 138.96 83.5) (end 147.1765 91.7165) (width 0.2) (layer "F.Cu") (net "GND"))
 (segment (start 168.699895 91.7165) (end 169.322 92.338605) (width 0.2) (layer "F.Cu") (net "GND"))
 (segment (start 169.7385 104) (end 157.318 104) (width 0.2) (layer "F.Cu") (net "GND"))
 (segment (start 147.1765 91.7165) (end 168.699895 91.7165) (width 0.2) (layer "F.Cu") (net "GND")))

